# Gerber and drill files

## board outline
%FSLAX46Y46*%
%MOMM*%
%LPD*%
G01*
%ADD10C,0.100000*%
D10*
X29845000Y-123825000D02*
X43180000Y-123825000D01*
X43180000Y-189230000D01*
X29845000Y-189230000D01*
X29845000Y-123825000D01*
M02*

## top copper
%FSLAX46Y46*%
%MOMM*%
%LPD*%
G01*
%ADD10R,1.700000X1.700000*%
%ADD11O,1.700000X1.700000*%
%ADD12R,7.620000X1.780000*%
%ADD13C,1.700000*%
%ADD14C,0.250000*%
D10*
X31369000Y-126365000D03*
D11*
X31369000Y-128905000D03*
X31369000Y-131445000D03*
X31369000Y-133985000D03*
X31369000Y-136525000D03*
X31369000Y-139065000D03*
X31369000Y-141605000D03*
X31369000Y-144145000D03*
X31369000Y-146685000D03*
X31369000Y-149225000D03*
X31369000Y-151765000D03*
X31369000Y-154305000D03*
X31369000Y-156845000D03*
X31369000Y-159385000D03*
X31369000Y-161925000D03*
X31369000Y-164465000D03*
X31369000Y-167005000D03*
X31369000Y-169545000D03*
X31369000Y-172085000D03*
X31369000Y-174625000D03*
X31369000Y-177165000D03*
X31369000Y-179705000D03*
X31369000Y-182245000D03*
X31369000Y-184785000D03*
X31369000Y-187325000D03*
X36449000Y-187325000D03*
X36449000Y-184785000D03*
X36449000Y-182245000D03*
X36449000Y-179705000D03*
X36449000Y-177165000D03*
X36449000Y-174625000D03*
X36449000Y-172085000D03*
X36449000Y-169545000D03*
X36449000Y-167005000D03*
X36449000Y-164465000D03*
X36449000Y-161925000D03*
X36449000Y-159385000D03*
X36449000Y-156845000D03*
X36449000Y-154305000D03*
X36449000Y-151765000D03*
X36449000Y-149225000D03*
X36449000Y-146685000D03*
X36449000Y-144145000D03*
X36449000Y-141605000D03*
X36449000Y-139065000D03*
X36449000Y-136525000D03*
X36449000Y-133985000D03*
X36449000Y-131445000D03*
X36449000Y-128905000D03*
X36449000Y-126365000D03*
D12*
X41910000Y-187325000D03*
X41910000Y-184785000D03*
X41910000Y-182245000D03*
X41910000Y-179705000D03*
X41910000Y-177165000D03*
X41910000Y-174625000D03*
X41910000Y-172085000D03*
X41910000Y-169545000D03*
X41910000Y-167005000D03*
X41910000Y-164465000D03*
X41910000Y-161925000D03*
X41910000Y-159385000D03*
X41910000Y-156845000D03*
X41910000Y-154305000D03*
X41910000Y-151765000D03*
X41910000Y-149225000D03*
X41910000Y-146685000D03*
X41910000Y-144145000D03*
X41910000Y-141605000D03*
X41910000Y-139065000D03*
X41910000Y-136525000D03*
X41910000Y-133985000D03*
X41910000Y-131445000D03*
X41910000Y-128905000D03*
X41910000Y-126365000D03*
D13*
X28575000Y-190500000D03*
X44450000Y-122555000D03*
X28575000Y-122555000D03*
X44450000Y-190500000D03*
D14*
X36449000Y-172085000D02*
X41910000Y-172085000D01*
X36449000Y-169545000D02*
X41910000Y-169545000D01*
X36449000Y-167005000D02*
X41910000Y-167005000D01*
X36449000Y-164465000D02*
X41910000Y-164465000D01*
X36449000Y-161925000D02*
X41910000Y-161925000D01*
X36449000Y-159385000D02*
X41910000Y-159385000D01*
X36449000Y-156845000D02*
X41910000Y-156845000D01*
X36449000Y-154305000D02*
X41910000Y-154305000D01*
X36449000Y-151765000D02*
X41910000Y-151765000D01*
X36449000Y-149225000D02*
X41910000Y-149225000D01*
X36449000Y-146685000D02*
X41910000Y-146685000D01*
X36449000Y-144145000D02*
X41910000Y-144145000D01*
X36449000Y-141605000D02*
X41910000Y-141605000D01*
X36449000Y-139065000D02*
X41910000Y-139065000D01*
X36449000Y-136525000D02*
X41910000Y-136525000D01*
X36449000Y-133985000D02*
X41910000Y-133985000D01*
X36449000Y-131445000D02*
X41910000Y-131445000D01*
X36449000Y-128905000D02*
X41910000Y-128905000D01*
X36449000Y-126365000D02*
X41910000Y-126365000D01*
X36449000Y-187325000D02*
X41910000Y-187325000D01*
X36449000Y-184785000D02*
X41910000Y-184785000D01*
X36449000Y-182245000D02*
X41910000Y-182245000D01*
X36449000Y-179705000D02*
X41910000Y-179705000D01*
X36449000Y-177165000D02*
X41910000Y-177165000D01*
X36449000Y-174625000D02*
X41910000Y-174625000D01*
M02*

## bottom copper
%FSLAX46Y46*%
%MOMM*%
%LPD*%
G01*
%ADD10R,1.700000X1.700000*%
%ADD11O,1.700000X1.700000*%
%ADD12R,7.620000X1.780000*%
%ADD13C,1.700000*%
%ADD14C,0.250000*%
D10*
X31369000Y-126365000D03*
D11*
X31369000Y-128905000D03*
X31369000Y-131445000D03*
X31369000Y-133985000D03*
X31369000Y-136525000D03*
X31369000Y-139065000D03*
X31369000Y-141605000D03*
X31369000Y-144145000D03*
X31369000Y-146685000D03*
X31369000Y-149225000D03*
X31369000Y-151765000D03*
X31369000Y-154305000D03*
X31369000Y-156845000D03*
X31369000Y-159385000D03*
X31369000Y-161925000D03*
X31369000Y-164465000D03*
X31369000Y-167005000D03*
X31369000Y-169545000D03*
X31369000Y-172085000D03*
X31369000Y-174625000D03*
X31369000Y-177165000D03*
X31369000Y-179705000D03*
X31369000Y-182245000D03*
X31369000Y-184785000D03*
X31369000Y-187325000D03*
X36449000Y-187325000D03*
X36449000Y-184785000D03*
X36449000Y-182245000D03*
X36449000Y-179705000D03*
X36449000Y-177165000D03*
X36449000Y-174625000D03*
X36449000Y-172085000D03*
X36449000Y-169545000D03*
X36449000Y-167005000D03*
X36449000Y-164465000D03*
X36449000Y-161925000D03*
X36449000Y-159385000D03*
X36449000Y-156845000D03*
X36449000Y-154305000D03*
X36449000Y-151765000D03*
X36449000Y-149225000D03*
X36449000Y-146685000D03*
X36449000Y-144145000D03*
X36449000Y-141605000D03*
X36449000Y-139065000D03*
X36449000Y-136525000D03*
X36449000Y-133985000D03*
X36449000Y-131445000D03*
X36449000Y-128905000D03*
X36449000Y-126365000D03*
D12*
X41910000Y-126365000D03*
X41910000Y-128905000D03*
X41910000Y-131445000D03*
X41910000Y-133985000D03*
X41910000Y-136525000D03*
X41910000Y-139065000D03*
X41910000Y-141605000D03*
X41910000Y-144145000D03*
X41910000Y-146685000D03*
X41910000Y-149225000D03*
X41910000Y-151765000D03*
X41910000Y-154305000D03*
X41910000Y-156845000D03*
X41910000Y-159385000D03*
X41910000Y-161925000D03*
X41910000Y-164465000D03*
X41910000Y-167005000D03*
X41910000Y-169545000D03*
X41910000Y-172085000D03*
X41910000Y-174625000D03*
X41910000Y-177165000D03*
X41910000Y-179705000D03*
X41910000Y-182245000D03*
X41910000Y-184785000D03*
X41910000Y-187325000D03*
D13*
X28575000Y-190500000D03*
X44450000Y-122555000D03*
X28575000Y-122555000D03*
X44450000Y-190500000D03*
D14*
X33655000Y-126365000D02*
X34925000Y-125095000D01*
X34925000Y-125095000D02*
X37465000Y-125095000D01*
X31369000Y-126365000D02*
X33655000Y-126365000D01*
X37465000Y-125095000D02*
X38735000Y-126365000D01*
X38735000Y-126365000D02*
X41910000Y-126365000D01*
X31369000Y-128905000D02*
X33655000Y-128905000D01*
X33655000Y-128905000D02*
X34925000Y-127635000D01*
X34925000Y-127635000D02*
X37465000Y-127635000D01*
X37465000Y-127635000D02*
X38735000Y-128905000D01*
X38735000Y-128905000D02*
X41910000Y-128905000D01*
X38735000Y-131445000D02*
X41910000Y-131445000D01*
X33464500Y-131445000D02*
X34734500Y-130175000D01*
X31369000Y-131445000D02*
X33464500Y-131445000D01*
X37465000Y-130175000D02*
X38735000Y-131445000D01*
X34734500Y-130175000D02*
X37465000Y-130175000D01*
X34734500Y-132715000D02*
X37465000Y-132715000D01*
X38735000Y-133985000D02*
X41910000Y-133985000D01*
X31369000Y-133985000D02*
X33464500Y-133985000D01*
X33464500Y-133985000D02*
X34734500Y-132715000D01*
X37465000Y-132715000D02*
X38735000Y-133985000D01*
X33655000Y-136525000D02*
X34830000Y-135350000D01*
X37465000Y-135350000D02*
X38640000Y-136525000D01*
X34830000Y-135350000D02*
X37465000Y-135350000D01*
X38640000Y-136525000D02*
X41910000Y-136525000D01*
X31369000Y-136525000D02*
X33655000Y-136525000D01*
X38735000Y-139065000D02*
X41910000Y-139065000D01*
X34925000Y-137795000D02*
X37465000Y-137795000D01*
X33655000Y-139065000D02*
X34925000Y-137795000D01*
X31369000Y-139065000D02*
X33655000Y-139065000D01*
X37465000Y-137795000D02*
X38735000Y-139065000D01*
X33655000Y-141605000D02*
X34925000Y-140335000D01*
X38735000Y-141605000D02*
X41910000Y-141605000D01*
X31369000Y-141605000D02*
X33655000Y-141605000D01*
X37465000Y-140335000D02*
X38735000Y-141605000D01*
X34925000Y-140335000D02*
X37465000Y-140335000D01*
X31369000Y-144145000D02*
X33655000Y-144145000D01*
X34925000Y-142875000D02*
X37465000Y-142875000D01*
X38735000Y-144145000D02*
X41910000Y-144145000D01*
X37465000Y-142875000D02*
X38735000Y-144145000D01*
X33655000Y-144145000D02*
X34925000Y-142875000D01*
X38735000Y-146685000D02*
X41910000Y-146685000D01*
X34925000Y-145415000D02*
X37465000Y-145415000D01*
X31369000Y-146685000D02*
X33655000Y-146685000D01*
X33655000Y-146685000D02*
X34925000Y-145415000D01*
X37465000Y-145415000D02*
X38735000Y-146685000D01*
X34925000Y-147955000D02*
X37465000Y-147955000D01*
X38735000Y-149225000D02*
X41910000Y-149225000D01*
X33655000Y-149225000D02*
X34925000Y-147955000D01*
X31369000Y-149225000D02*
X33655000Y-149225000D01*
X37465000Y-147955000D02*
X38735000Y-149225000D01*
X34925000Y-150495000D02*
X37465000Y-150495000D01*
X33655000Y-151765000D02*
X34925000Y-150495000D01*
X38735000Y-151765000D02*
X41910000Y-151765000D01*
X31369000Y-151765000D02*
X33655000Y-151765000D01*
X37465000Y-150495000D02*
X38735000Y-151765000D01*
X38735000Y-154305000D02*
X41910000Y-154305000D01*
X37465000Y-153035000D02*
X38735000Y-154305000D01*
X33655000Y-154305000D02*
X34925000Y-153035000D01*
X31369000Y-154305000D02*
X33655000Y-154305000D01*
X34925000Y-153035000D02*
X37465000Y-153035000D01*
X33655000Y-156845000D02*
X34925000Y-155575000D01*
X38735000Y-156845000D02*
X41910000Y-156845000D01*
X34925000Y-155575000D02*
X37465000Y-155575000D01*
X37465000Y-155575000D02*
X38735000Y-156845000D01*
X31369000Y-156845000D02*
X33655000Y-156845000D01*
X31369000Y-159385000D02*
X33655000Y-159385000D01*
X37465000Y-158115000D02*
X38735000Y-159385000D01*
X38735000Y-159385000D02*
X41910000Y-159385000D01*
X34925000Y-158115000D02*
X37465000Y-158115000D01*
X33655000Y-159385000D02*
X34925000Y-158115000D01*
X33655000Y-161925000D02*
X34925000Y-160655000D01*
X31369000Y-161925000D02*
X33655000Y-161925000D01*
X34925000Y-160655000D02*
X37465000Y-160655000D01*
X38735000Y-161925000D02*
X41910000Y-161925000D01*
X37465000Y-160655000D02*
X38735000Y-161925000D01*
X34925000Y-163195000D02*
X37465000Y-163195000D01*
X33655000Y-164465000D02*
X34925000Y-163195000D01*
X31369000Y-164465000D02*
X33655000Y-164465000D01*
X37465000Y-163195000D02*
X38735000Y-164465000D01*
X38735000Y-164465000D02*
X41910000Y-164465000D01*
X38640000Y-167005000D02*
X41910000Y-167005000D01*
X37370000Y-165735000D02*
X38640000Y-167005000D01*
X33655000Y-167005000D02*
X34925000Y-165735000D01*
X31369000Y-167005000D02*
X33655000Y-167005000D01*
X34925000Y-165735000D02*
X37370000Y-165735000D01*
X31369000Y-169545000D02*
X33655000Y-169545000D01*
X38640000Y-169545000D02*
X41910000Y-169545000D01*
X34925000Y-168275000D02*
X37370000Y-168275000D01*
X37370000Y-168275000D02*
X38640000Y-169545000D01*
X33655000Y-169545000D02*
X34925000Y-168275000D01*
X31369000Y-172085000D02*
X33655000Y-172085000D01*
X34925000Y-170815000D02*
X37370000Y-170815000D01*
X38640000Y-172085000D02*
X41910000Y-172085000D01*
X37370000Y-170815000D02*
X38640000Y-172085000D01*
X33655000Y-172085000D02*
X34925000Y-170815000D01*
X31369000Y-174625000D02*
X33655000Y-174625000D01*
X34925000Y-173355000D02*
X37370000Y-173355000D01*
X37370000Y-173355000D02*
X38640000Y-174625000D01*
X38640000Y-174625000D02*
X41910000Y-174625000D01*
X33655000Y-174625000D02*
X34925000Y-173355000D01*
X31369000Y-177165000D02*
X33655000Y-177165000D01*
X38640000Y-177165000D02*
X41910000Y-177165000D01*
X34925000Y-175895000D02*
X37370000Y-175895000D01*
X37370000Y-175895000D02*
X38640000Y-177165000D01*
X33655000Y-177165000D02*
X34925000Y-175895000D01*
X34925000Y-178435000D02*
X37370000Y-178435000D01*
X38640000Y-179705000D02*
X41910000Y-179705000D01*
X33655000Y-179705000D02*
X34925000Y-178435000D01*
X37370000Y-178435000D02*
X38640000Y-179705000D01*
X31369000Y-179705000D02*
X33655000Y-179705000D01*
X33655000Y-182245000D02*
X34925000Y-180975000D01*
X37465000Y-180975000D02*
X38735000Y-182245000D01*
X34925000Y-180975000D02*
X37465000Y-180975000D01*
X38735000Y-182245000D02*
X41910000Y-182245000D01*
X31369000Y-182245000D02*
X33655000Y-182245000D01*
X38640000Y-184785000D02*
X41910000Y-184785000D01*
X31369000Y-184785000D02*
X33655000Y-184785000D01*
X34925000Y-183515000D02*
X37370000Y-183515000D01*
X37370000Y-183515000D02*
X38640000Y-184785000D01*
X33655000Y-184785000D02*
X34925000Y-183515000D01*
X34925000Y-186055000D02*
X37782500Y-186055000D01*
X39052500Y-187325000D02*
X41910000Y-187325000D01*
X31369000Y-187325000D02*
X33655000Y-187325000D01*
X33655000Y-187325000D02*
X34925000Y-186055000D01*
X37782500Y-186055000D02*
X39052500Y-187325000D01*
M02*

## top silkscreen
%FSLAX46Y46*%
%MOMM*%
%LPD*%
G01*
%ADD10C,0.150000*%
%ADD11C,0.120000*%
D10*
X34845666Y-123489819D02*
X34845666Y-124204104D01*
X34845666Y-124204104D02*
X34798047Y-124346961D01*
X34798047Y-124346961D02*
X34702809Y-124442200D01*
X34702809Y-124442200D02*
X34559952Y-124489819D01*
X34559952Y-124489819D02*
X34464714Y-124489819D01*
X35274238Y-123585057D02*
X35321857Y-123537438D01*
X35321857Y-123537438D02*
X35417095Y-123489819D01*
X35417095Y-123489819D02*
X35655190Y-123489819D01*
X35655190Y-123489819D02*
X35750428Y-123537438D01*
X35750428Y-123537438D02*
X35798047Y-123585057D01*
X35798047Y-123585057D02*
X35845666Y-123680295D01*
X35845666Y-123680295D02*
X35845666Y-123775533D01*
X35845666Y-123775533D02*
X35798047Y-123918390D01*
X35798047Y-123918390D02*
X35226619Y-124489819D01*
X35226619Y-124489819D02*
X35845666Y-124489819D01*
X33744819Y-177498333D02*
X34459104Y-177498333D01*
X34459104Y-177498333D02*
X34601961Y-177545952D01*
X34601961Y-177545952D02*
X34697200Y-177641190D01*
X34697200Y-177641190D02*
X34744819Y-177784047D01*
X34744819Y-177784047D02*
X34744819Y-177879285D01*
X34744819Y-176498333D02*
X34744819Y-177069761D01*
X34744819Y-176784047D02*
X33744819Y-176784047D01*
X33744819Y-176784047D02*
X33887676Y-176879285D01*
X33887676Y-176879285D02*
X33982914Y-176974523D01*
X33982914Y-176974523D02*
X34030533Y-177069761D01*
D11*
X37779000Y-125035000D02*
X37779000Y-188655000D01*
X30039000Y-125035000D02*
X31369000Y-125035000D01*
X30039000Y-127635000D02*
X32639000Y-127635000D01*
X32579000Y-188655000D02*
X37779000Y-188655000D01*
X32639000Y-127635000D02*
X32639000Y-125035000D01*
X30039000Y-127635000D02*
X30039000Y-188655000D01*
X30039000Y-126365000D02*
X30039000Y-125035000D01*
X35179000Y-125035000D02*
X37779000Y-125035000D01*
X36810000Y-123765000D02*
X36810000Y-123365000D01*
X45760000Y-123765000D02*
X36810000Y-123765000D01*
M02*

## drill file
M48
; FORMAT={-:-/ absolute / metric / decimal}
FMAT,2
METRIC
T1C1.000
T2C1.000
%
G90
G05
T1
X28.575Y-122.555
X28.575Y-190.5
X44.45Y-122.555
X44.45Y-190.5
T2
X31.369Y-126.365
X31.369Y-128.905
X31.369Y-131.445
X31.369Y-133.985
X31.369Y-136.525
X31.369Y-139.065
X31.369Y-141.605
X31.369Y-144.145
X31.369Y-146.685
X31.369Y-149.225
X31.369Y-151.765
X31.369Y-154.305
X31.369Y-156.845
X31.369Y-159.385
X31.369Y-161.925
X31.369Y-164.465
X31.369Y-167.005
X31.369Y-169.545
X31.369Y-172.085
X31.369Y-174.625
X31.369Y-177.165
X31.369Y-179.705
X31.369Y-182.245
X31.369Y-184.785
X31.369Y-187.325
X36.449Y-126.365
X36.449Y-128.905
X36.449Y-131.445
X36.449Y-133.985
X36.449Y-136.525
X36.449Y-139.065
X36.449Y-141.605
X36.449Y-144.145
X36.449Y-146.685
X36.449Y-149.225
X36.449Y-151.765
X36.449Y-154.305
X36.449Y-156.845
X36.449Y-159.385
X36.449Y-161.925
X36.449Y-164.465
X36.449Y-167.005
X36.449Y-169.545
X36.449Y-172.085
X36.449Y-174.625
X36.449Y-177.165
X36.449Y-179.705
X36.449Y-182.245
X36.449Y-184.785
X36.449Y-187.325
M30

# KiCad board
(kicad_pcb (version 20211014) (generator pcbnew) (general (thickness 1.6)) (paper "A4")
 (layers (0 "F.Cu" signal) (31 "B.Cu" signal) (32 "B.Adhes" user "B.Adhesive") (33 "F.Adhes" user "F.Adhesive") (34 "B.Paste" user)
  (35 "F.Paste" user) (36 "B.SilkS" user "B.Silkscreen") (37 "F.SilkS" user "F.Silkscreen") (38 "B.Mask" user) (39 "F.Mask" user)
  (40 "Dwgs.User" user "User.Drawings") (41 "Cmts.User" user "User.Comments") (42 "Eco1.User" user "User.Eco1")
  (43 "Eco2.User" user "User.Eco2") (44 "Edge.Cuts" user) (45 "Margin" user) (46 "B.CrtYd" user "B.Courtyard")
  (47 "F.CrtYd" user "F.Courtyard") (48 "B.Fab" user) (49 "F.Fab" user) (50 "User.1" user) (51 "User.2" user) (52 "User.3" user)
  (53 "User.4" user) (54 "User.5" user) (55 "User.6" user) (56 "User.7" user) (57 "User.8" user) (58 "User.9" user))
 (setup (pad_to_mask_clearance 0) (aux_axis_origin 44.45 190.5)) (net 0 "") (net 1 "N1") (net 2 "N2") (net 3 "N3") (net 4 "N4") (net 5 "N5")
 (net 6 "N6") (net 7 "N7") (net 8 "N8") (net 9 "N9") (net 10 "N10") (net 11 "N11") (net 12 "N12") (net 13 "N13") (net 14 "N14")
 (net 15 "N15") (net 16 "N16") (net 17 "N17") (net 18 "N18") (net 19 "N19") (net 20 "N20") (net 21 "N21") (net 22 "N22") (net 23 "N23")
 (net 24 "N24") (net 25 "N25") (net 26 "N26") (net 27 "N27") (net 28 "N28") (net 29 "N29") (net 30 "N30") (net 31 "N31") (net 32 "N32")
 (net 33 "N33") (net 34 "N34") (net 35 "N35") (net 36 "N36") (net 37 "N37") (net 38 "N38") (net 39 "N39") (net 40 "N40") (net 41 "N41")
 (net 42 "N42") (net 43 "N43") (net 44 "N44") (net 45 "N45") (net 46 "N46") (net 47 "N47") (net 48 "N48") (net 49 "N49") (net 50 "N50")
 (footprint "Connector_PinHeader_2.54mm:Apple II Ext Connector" (layer "F.Cu") (at 31.369 126.365)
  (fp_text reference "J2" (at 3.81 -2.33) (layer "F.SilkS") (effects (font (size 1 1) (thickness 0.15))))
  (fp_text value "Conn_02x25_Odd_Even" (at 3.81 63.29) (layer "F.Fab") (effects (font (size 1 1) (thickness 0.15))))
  (fp_line (start 6.41 -1.33) (end 6.41 62.29) (layer "F.SilkS") (width 0.12))
  (fp_line (start -1.33 -1.33) (end 0 -1.33) (layer "F.SilkS") (width 0.12))
  (fp_line (start -1.33 1.27) (end 1.27 1.27) (layer "F.SilkS") (width 0.12))
  (fp_line (start 1.21 62.29) (end 6.41 62.29) (layer "F.SilkS") (width 0.12))
  (fp_line (start 1.27 1.27) (end 1.27 -1.33) (layer "F.SilkS") (width 0.12))
  (fp_line (start -1.33 1.27) (end -1.33 62.29) (layer "F.SilkS") (width 0.12))
  (fp_line (start -1.33 0) (end -1.33 -1.33) (layer "F.SilkS") (width 0.12))
  (fp_line (start 3.81 -1.33) (end 6.41 -1.33) (layer "F.SilkS") (width 0.12))
  (pad "1" thru_hole rect (at 0 0) (size 1.7 1.7) (drill 1) (layers *.Cu *.Mask) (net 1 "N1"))
  (pad "2" thru_hole oval (at 0 2.54) (size 1.7 1.7) (drill 1) (layers *.Cu *.Mask) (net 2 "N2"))
  (pad "3" thru_hole oval (at 0 5.08) (size 1.7 1.7) (drill 1) (layers *.Cu *.Mask) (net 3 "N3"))
  (pad "4" thru_hole oval (at 0 7.62) (size 1.7 1.7) (drill 1) (layers *.Cu *.Mask) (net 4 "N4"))
  (pad "5" thru_hole oval (at 0 10.16) (size 1.7 1.7) (drill 1) (layers *.Cu *.Mask) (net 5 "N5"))
  (pad "6" thru_hole oval (at 0 12.7) (size 1.7 1.7) (drill 1) (layers *.Cu *.Mask) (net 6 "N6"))
  (pad "7" thru_hole oval (at 0 15.24) (size 1.7 1.7) (drill 1) (layers *.Cu *.Mask) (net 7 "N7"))
  (pad "8" thru_hole oval (at 0 17.78) (size 1.7 1.7) (drill 1) (layers *.Cu *.Mask) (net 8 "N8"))
  (pad "9" thru_hole oval (at 0 20.32) (size 1.7 1.7) (drill 1) (layers *.Cu *.Mask) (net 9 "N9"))
  (pad "10" thru_hole oval (at 0 22.86) (size 1.7 1.7) (drill 1) (layers *.Cu *.Mask) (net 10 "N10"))
  (pad "11" thru_hole oval (at 0 25.4) (size 1.7 1.7) (drill 1) (layers *.Cu *.Mask) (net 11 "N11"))
  (pad "12" thru_hole oval (at 0 27.94) (size 1.7 1.7) (drill 1) (layers *.Cu *.Mask) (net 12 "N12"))
  (pad "13" thru_hole oval (at 0 30.48) (size 1.7 1.7) (drill 1) (layers *.Cu *.Mask) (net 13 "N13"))
  (pad "14" thru_hole oval (at 0 33.02) (size 1.7 1.7) (drill 1) (layers *.Cu *.Mask) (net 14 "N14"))
  (pad "15" thru_hole oval (at 0 35.56) (size 1.7 1.7) (drill 1) (layers *.Cu *.Mask) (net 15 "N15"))
  (pad "16" thru_hole oval (at 0 38.1) (size 1.7 1.7) (drill 1) (layers *.Cu *.Mask) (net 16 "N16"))
  (pad "17" thru_hole oval (at 0 40.64) (size 1.7 1.7) (drill 1) (layers *.Cu *.Mask) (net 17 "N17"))
  (pad "18" thru_hole oval (at 0 43.18) (size 1.7 1.7) (drill 1) (layers *.Cu *.Mask) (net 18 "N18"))
  (pad "19" thru_hole oval (at 0 45.72) (size 1.7 1.7) (drill 1) (layers *.Cu *.Mask) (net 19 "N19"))
  (pad "20" thru_hole oval (at 0 48.26) (size 1.7 1.7) (drill 1) (layers *.Cu *.Mask) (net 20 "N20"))
  (pad "21" thru_hole oval (at 0 50.8) (size 1.7 1.7) (drill 1) (layers *.Cu *.Mask) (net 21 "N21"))
  (pad "22" thru_hole oval (at 0 53.34) (size 1.7 1.7) (drill 1) (layers *.Cu *.Mask) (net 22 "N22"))
  (pad "23" thru_hole oval (at 0 55.88) (size 1.7 1.7) (drill 1) (layers *.Cu *.Mask) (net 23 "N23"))
  (pad "24" thru_hole oval (at 0 58.42) (size 1.7 1.7) (drill 1) (layers *.Cu *.Mask) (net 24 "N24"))
  (pad "25" thru_hole oval (at 0 60.96) (size 1.7 1.7) (drill 1) (layers *.Cu *.Mask) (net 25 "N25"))
  (pad "26" thru_hole oval (at 5.08 60.96 180) (size 1.7 1.7) (drill 1) (layers *.Cu *.Mask) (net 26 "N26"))
  (pad "27" thru_hole oval (at 5.08 58.42 180) (size 1.7 1.7) (drill 1) (layers *.Cu *.Mask) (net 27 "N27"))
  (pad "28" thru_hole oval (at 5.08 55.88 180) (size 1.7 1.7) (drill 1) (layers *.Cu *.Mask) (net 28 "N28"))
  (pad "29" thru_hole oval (at 5.08 53.34 180) (size 1.7 1.7) (drill 1) (layers *.Cu *.Mask) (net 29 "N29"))
  (pad "30" thru_hole oval (at 5.08 50.8 180) (size 1.7 1.7) (drill 1) (layers *.Cu *.Mask) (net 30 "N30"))
  (pad "31" thru_hole oval (at 5.08 48.26 180) (size 1.7 1.7) (drill 1) (layers *.Cu *.Mask) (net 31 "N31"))
  (pad "32" thru_hole oval (at 5.08 45.72 180) (size 1.7 1.7) (drill 1) (layers *.Cu *.Mask) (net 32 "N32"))
  (pad "33" thru_hole oval (at 5.08 43.18 180) (size 1.7 1.7) (drill 1) (layers *.Cu *.Mask) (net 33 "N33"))
  (pad "34" thru_hole oval (at 5.08 40.64 180) (size 1.7 1.7) (drill 1) (layers *.Cu *.Mask) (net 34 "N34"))
  (pad "35" thru_hole oval (at 5.08 38.1 180) (size 1.7 1.7) (drill 1) (layers *.Cu *.Mask) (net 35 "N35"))
  (pad "36" thru_hole oval (at 5.08 35.56 180) (size 1.7 1.7) (drill 1) (layers *.Cu *.Mask) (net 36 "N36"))
  (pad "37" thru_hole oval (at 5.08 33.02 180) (size 1.7 1.7) (drill 1) (layers *.Cu *.Mask) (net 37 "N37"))
  (pad "38" thru_hole oval (at 5.08 30.48 180) (size 1.7 1.7) (drill 1) (layers *.Cu *.Mask) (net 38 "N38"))
  (pad "39" thru_hole oval (at 5.08 27.94 180) (size 1.7 1.7) (drill 1) (layers *.Cu *.Mask) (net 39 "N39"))
  (pad "40" thru_hole oval (at 5.08 25.4 180) (size 1.7 1.7) (drill 1) (layers *.Cu *.Mask) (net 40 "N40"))
  (pad "41" thru_hole oval (at 5.08 22.86 180) (size 1.7 1.7) (drill 1) (layers *.Cu *.Mask) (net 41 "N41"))
  (pad "42" thru_hole oval (at 5.08 20.32 180) (size 1.7 1.7) (drill 1) (layers *.Cu *.Mask) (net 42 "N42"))
  (pad "43" thru_hole oval (at 5.08 17.78 180) (size 1.7 1.7) (drill 1) (layers *.Cu *.Mask) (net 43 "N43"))
  (pad "44" thru_hole oval (at 5.08 15.24 180) (size 1.7 1.7) (drill 1) (layers *.Cu *.Mask) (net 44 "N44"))
  (pad "45" thru_hole oval (at 5.08 12.7 180) (size 1.7 1.7) (drill 1) (layers *.Cu *.Mask) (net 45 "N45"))
  (pad "46" thru_hole oval (at 5.08 10.16 180) (size 1.7 1.7) (drill 1) (layers *.Cu *.Mask) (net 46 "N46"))
  (pad "47" thru_hole oval (at 5.08 7.62 180) (size 1.7 1.7) (drill 1) (layers *.Cu *.Mask) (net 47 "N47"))
  (pad "48" thru_hole oval (at 5.08 5.08 180) (size 1.7 1.7) (drill 1) (layers *.Cu *.Mask) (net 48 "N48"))
  (pad "49" thru_hole oval (at 5.08 2.54 180) (size 1.7 1.7) (drill 1) (layers *.Cu *.Mask) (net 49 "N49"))
  (pad "50" thru_hole oval (at 5.08 0 180) (size 1.7 1.7) (drill 1) (layers *.Cu *.Mask) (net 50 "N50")))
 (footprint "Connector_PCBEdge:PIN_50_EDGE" (layer "F.Cu") (at 41.91 126.365 90)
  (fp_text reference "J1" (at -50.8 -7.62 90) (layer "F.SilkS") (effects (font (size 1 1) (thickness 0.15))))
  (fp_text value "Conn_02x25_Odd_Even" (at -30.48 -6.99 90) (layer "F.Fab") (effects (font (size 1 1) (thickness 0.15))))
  (fp_line (start 2.6 -5.1) (end 3 -5.1) (layer "F.SilkS") (width 0.12))
  (fp_line (start 2.6 3.85) (end 2.6 -5.1) (layer "F.SilkS") (width 0.12))
  (pad "1" connect rect (at 0 0 90) (size 1.78 7.62) (layers "B.Cu" "B.Mask") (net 1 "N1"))
  (pad "2" connect rect (at -2.54 0 90) (size 1.78 7.62) (layers "B.Cu" "B.Mask") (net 2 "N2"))
  (pad "3" connect rect (at -5.08 0 90) (size 1.78 7.62) (layers "B.Cu" "B.Mask") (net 3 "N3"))
  (pad "4" connect rect (at -7.62 0 90) (size 1.78 7.62) (layers "B.Cu" "B.Mask") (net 4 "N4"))
  (pad "5" connect rect (at -10.16 0 90) (size 1.78 7.62) (layers "B.Cu" "B.Mask") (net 5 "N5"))
  (pad "6" connect rect (at -12.7 0 90) (size 1.78 7.62) (layers "B.Cu" "B.Mask") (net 6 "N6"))
  (pad "7" connect rect (at -15.24 0 90) (size 1.78 7.62) (layers "B.Cu" "B.Mask") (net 7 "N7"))
  (pad "8" connect rect (at -17.78 0 90) (size 1.78 7.62) (layers "B.Cu" "B.Mask") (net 8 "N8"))
  (pad "9" connect rect (at -20.32 0 90) (size 1.78 7.62) (layers "B.Cu" "B.Mask") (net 9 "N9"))
  (pad "10" connect rect (at -22.86 0 90) (size 1.78 7.62) (layers "B.Cu" "B.Mask") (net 10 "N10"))
  (pad "11" connect rect (at -25.4 0 90) (size 1.78 7.62) (layers "B.Cu" "B.Mask") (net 11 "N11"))
  (pad "12" connect rect (at -27.94 0 90) (size 1.78 7.62) (layers "B.Cu" "B.Mask") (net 12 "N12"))
  (pad "13" connect rect (at -30.48 0 90) (size 1.78 7.62) (layers "B.Cu" "B.Mask") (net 13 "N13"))
  (pad "14" connect rect (at -33.02 0 90) (size 1.78 7.62) (layers "B.Cu" "B.Mask") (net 14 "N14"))
  (pad "15" connect rect (at -35.56 0 90) (size 1.78 7.62) (layers "B.Cu" "B.Mask") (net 15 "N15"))
  (pad "16" connect rect (at -38.1 0 90) (size 1.78 7.62) (layers "B.Cu" "B.Mask") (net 16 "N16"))
  (pad "17" connect rect (at -40.64 0 90) (size 1.78 7.62) (layers "B.Cu" "B.Mask") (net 17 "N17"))
  (pad "18" connect rect (at -43.18 0 90) (size 1.78 7.62) (layers "B.Cu" "B.Mask") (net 18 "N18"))
  (pad "19" connect rect (at -45.72 0 90) (size 1.78 7.62) (layers "B.Cu" "B.Mask") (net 19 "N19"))
  (pad "20" connect rect (at -48.26 0 90) (size 1.78 7.62) (layers "B.Cu" "B.Mask") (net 20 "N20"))
  (pad "21" connect rect (at -50.8 0 90) (size 1.78 7.62) (layers "B.Cu" "B.Mask") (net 21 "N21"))
  (pad "22" connect rect (at -53.34 0 90) (size 1.78 7.62) (layers "B.Cu" "B.Mask") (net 22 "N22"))
  (pad "23" connect rect (at -55.88 0 90) (size 1.78 7.62) (layers "B.Cu" "B.Mask") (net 23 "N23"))
  (pad "24" connect rect (at -58.42 0 90) (size 1.78 7.62) (layers "B.Cu" "B.Mask") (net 24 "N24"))
  (pad "25" connect rect (at -60.96 0 90) (size 1.78 7.62) (layers "B.Cu" "B.Mask") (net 25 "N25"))
  (pad "26" connect rect (at -60.96 0 90) (size 1.78 7.62) (layers "F.Cu" "F.Mask") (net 26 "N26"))
  (pad "27" connect rect (at -58.42 0 90) (size 1.78 7.62) (layers "F.Cu" "F.Mask") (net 27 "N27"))
  (pad "28" connect rect (at -55.88 0 90) (size 1.78 7.62) (layers "F.Cu" "F.Mask") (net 28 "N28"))
  (pad "29" connect rect (at -53.34 0 90) (size 1.78 7.62) (layers "F.Cu" "F.Mask") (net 29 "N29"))
  (pad "30" connect rect (at -50.8 0 90) (size 1.78 7.62) (layers "F.Cu" "F.Mask") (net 30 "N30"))
  (pad "31" connect rect (at -48.26 0 90) (size 1.78 7.62) (layers "F.Cu" "F.Mask") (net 31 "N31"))
  (pad "32" connect rect (at -45.72 0 90) (size 1.78 7.62) (layers "F.Cu" "F.Mask") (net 32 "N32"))
  (pad "33" connect rect (at -43.18 0 90) (size 1.78 7.62) (layers "F.Cu" "F.Mask") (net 33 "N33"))
  (pad "34" connect rect (at -40.64 0 90) (size 1.78 7.62) (layers "F.Cu" "F.Mask") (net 34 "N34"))
  (pad "35" connect rect (at -38.1 0 90) (size 1.78 7.62) (layers "F.Cu" "F.Mask") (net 35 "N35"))
  (pad "36" connect rect (at -35.56 0 90) (size 1.78 7.62) (layers "F.Cu" "F.Mask") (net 36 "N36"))
  (pad "37" connect rect (at -33.02 0 90) (size 1.78 7.62) (layers "F.Cu" "F.Mask") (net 37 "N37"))
  (pad "38" connect rect (at -30.48 0 90) (size 1.78 7.62) (layers "F.Cu" "F.Mask") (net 38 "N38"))
  (pad "39" connect rect (at -27.94 0 90) (size 1.78 7.62) (layers "F.Cu" "F.Mask") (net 39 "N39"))
  (pad "40" connect rect (at -25.4 0 90) (size 1.78 7.62) (layers "F.Cu" "F.Mask") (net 40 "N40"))
  (pad "41" connect rect (at -22.86 0 90) (size 1.78 7.62) (layers "F.Cu" "F.Mask") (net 41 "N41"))
  (pad "42" connect rect (at -20.32 0 90) (size 1.78 7.62) (layers "F.Cu" "F.Mask") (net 42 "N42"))
  (pad "43" connect rect (at -17.78 0 90) (size 1.78 7.62) (layers "F.Cu" "F.Mask") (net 43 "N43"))
  (pad "44" connect rect (at -15.24 0 90) (size 1.78 7.62) (layers "F.Cu" "F.Mask") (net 44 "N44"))
  (pad "45" connect rect (at -12.7 0 90) (size 1.78 7.62) (layers "F.Cu" "F.Mask") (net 45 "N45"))
  (pad "46" connect rect (at -10.16 0 90) (size 1.78 7.62) (layers "F.Cu" "F.Mask") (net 46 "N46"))
  (pad "47" connect rect (at -7.62 0 90) (size 1.78 7.62) (layers "F.Cu" "F.Mask") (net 47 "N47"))
  (pad "48" connect rect (at -5.08 0 90) (size 1.78 7.62) (layers "F.Cu" "F.Mask") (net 48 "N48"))
  (pad "49" connect rect (at -2.54 0 90) (size 1.78 7.62) (layers "F.Cu" "F.Mask") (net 49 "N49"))
  (pad "50" connect rect (at 0 0 90) (size 1.78 7.62) (layers "F.Cu" "F.Mask") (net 50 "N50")))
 (gr_rect (start 29.845 123.825) (end 43.18 189.23) (layer "Edge.Cuts") (width 0.1) (fill none))
 (via (at 28.575 190.5) (size 1.7) (drill 1) (layers "F.Cu" "B.Cu") (free) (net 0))
 (via (at 44.45 122.555) (size 1.7) (drill 1) (layers "F.Cu" "B.Cu") (free) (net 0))
 (via (at 28.575 122.555) (size 1.7) (drill 1) (layers "F.Cu" "B.Cu") (free) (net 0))
 (via (at 44.45 190.5) (size 1.7) (drill 1) (layers "F.Cu" "B.Cu") (free) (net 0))
 (segment (start 33.655 126.365) (end 34.925 125.095) (width 0.25) (layer "B.Cu") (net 1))
 (segment (start 34.925 125.095) (end 37.465 125.095) (width 0.25) (layer "B.Cu") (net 1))
 (segment (start 31.369 126.365) (end 33.655 126.365) (width 0.25) (layer "B.Cu") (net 1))
 (segment (start 37.465 125.095) (end 38.735 126.365) (width 0.25) (layer "B.Cu") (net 1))
 (segment (start 38.735 126.365) (end 41.91 126.365) (width 0.25) (layer "B.Cu") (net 1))
 (segment (start 31.369 128.905) (end 33.655 128.905) (width 0.25) (layer "B.Cu") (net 2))
 (segment (start 33.655 128.905) (end 34.925 127.635) (width 0.25) (layer "B.Cu") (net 2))
 (segment (start 34.925 127.635) (end 37.465 127.635) (width 0.25) (layer "B.Cu") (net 2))
 (segment (start 37.465 127.635) (end 38.735 128.905) (width 0.25) (layer "B.Cu") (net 2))
 (segment (start 38.735 128.905) (end 41.91 128.905) (width 0.25) (layer "B.Cu") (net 2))
 (segment (start 38.735 131.445) (end 41.91 131.445) (width 0.25) (layer "B.Cu") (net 3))
 (segment (start 33.4645 131.445) (end 34.7345 130.175) (width 0.25) (layer "B.Cu") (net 3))
 (segment (start 31.369 131.445) (end 33.4645 131.445) (width 0.25) (layer "B.Cu") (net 3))
 (segment (start 37.465 130.175) (end 38.735 131.445) (width 0.25) (layer "B.Cu") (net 3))
 (segment (start 34.7345 130.175) (end 37.465 130.175) (width 0.25) (layer "B.Cu") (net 3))
 (segment (start 34.7345 132.715) (end 37.465 132.715) (width 0.25) (layer "B.Cu") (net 4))
 (segment (start 38.735 133.985) (end 41.91 133.985) (width 0.25) (layer "B.Cu") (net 4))
 (segment (start 31.369 133.985) (end 33.4645 133.985) (width 0.25) (layer "B.Cu") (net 4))
 (segment (start 33.4645 133.985) (end 34.7345 132.715) (width 0.25) (layer "B.Cu") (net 4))
 (segment (start 37.465 132.715) (end 38.735 133.985) (width 0.25) (layer "B.Cu") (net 4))
 (segment (start 33.655 136.525) (end 34.83 135.35) (width 0.25) (layer "B.Cu") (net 5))
 (segment (start 37.465 135.35) (end 38.64 136.525) (width 0.25) (layer "B.Cu") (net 5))
 (segment (start 34.83 135.35) (end 37.465 135.35) (width 0.25) (layer "B.Cu") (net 5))
 (segment (start 38.64 136.525) (end 41.91 136.525) (width 0.25) (layer "B.Cu") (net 5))
 (segment (start 31.369 136.525) (end 33.655 136.525) (width 0.25) (layer "B.Cu") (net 5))
 (segment (start 38.735 139.065) (end 41.91 139.065) (width 0.25) (layer "B.Cu") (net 6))
 (segment (start 34.925 137.795) (end 37.465 137.795) (width 0.25) (layer "B.Cu") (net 6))
 (segment (start 33.655 139.065) (end 34.925 137.795) (width 0.25) (layer "B.Cu") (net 6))
 (segment (start 31.369 139.065) (end 33.655 139.065) (width 0.25) (layer "B.Cu") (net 6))
 (segment (start 37.465 137.795) (end 38.735 139.065) (width 0.25) (layer "B.Cu") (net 6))
 (segment (start 33.655 141.605) (end 34.925 140.335) (width 0.25) (layer "B.Cu") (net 7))
 (segment (start 38.735 141.605) (end 41.91 141.605) (width 0.25) (layer "B.Cu") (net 7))
 (segment (start 31.369 141.605) (end 33.655 141.605) (width 0.25) (layer "B.Cu") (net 7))
 (segment (start 37.465 140.335) (end 38.735 141.605) (width 0.25) (layer "B.Cu") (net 7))
 (segment (start 34.925 140.335) (end 37.465 140.335) (width 0.25) (layer "B.Cu") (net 7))
 (segment (start 31.369 144.145) (end 33.655 144.145) (width 0.25) (layer "B.Cu") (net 8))
 (segment (start 34.925 142.875) (end 37.465 142.875) (width 0.25) (layer "B.Cu") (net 8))
 (segment (start 38.735 144.145) (end 41.91 144.145) (width 0.25) (layer "B.Cu") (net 8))
 (segment (start 37.465 142.875) (end 38.735 144.145) (width 0.25) (layer "B.Cu") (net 8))
 (segment (start 33.655 144.145) (end 34.925 142.875) (width 0.25) (layer "B.Cu") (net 8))
 (segment (start 38.735 146.685) (end 41.91 146.685) (width 0.25) (layer "B.Cu") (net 9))
 (segment (start 34.925 145.415) (end 37.465 145.415) (width 0.25) (layer "B.Cu") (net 9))
 (segment (start 31.369 146.685) (end 33.655 146.685) (width 0.25) (layer "B.Cu") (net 9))
 (segment (start 33.655 146.685) (end 34.925 145.415) (width 0.25) (layer "B.Cu") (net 9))
 (segment (start 37.465 145.415) (end 38.735 146.685) (width 0.25) (layer "B.Cu") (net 9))
 (segment (start 34.925 147.955) (end 37.465 147.955) (width 0.25) (layer "B.Cu") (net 10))
 (segment (start 38.735 149.225) (end 41.91 149.225) (width 0.25) (layer "B.Cu") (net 10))
 (segment (start 33.655 149.225) (end 34.925 147.955) (width 0.25) (layer "B.Cu") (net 10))
 (segment (start 31.369 149.225) (end 33.655 149.225) (width 0.25) (layer "B.Cu") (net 10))
 (segment (start 37.465 147.955) (end 38.735 149.225) (width 0.25) (layer "B.Cu") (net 10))
 (segment (start 34.925 150.495) (end 37.465 150.495) (width 0.25) (layer "B.Cu") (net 11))
 (segment (start 33.655 151.765) (end 34.925 150.495) (width 0.25) (layer "B.Cu") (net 11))
 (segment (start 38.735 151.765) (end 41.91 151.765) (width 0.25) (layer "B.Cu") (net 11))
 (segment (start 31.369 151.765) (end 33.655 151.765) (width 0.25) (layer "B.Cu") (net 11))
 (segment (start 37.465 150.495) (end 38.735 151.765) (width 0.25) (layer "B.Cu") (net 11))
 (segment (start 38.735 154.305) (end 41.91 154.305) (width 0.25) (layer "B.Cu") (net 12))
 (segment (start 37.465 153.035) (end 38.735 154.305) (width 0.25) (layer "B.Cu") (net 12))
 (segment (start 33.655 154.305) (end 34.925 153.035) (width 0.25) (layer "B.Cu") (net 12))
 (segment (start 31.369 154.305) (end 33.655 154.305) (width 0.25) (layer "B.Cu") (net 12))
 (segment (start 34.925 153.035) (end 37.465 153.035) (width 0.25) (layer "B.Cu") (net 12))
 (segment (start 33.655 156.845) (end 34.925 155.575) (width 0.25) (layer "B.Cu") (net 13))
 (segment (start 38.735 156.845) (end 41.91 156.845) (width 0.25) (layer "B.Cu") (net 13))
 (segment (start 34.925 155.575) (end 37.465 155.575) (width 0.25) (layer "B.Cu") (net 13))
 (segment (start 37.465 155.575) (end 38.735 156.845) (width 0.25) (layer "B.Cu") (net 13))
 (segment (start 31.369 156.845) (end 33.655 156.845) (width 0.25) (layer "B.Cu") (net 13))
 (segment (start 31.369 159.385) (end 33.655 159.385) (width 0.25) (layer "B.Cu") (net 14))
 (segment (start 37.465 158.115) (end 38.735 159.385) (width 0.25) (layer "B.Cu") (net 14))
 (segment (start 38.735 159.385) (end 41.91 159.385) (width 0.25) (layer "B.Cu") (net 14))
 (segment (start 34.925 158.115) (end 37.465 158.115) (width 0.25) (layer "B.Cu") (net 14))
 (segment (start 33.655 159.385) (end 34.925 158.115) (width 0.25) (layer "B.Cu") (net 14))
 (segment (start 33.655 161.925) (end 34.925 160.655) (width 0.25) (layer "B.Cu") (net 15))
 (segment (start 31.369 161.925) (end 33.655 161.925) (width 0.25) (layer "B.Cu") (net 15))
 (segment (start 34.925 160.655) (end 37.465 160.655) (width 0.25) (layer "B.Cu") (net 15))
 (segment (start 38.735 161.925) (end 41.91 161.925) (width 0.25) (layer "B.Cu") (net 15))
 (segment (start 37.465 160.655) (end 38.735 161.925) (width 0.25) (layer "B.Cu") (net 15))
 (segment (start 34.925 163.195) (end 37.465 163.195) (width 0.25) (layer "B.Cu") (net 16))
 (segment (start 33.655 164.465) (end 34.925 163.195) (width 0.25) (layer "B.Cu") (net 16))
 (segment (start 31.369 164.465) (end 33.655 164.465) (width 0.25) (layer "B.Cu") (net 16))
 (segment (start 37.465 163.195) (end 38.735 164.465) (width 0.25) (layer "B.Cu") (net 16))
 (segment (start 38.735 164.465) (end 41.91 164.465) (width 0.25) (layer "B.Cu") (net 16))
 (segment (start 38.64 167.005) (end 41.91 167.005) (width 0.25) (layer "B.Cu") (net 17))
 (segment (start 37.37 165.735) (end 38.64 167.005) (width 0.25) (layer "B.Cu") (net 17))
 (segment (start 33.655 167.005) (end 34.925 165.735) (width 0.25) (layer "B.Cu") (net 17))
 (segment (start 31.369 167.005) (end 33.655 167.005) (width 0.25) (layer "B.Cu") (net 17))
 (segment (start 34.925 165.735) (end 37.37 165.735) (width 0.25) (layer "B.Cu") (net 17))
 (segment (start 31.369 169.545) (end 33.655 169.545) (width 0.25) (layer "B.Cu") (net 18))
 (segment (start 38.64 169.545) (end 41.91 169.545) (width 0.25) (layer "B.Cu") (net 18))
 (segment (start 34.925 168.275) (end 37.37 168.275) (width 0.25) (layer "B.Cu") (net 18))
 (segment (start 37.37 168.275) (end 38.64 169.545) (width 0.25) (layer "B.Cu") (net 18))
 (segment (start 33.655 169.545) (end 34.925 168.275) (width 0.25) (layer "B.Cu") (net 18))
 (segment (start 31.369 172.085) (end 33.655 172.085) (width 0.25) (layer "B.Cu") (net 19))
 (segment (start 34.925 170.815) (end 37.37 170.815) (width 0.25) (layer "B.Cu") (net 19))
 (segment (start 38.64 172.085) (end 41.91 172.085) (width 0.25) (layer "B.Cu") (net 19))
 (segment (start 37.37 170.815) (end 38.64 172.085) (width 0.25) (layer "B.Cu") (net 19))
 (segment (start 33.655 172.085) (end 34.925 170.815) (width 0.25) (layer "B.Cu") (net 19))
 (segment (start 31.369 174.625) (end 33.655 174.625) (width 0.25) (layer "B.Cu") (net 20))
 (segment (start 34.925 173.355) (end 37.37 173.355) (width 0.25) (layer "B.Cu") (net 20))
 (segment (start 37.37 173.355) (end 38.64 174.625) (width 0.25) (layer "B.Cu") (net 20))
 (segment (start 38.64 174.625) (end 41.91 174.625) (width 0.25) (layer "B.Cu") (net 20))
 (segment (start 33.655 174.625) (end 34.925 173.355) (width 0.25) (layer "B.Cu") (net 20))
 (segment (start 31.369 177.165) (end 33.655 177.165) (width 0.25) (layer "B.Cu") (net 21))
 (segment (start 38.64 177.165) (end 41.91 177.165) (width 0.25) (layer "B.Cu") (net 21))
 (segment (start 34.925 175.895) (end 37.37 175.895) (width 0.25) (layer "B.Cu") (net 21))
 (segment (start 37.37 175.895) (end 38.64 177.165) (width 0.25) (layer "B.Cu") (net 21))
 (segment (start 33.655 177.165) (end 34.925 175.895) (width 0.25) (layer "B.Cu") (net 21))
 (segment (start 34.925 178.435) (end 37.37 178.435) (width 0.25) (layer "B.Cu") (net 22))
 (segment (start 38.64 179.705) (end 41.91 179.705) (width 0.25) (layer "B.Cu") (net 22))
 (segment (start 33.655 179.705) (end 34.925 178.435) (width 0.25) (layer "B.Cu") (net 22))
 (segment (start 37.37 178.435) (end 38.64 179.705) (width 0.25) (layer "B.Cu") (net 22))
 (segment (start 31.369 179.705) (end 33.655 179.705) (width 0.25) (layer "B.Cu") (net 22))
 (segment (start 33.655 182.245) (end 34.925 180.975) (width 0.25) (layer "B.Cu") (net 23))
 (segment (start 37.465 180.975) (end 38.735 182.245) (width 0.25) (layer "B.Cu") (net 23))
 (segment (start 34.925 180.975) (end 37.465 180.975) (width 0.25) (layer "B.Cu") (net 23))
 (segment (start 38.735 182.245) (end 41.91 182.245) (width 0.25) (layer "B.Cu") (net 23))
 (segment (start 31.369 182.245) (end 33.655 182.245) (width 0.25) (layer "B.Cu") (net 23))
 (segment (start 38.64 184.785) (end 41.91 184.785) (width 0.25) (layer "B.Cu") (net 24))
 (segment (start 31.369 184.785) (end 33.655 184.785) (width 0.25) (layer "B.Cu") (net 24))
 (segment (start 34.925 183.515) (end 37.37 183.515) (width 0.25) (layer "B.Cu") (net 24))
 (segment (start 37.37 183.515) (end 38.64 184.785) (width 0.25) (layer "B.Cu") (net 24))
 (segment (start 33.655 184.785) (end 34.925 183.515) (width 0.25) (layer "B.Cu") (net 24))
 (segment (start 34.925 186.055) (end 37.7825 186.055) (width 0.25) (layer "B.Cu") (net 25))
 (segment (start 39.0525 187.325) (end 41.91 187.325) (width 0.25) (layer "B.Cu") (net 25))
 (segment (start 31.369 187.325) (end 33.655 187.325) (width 0.25) (layer "B.Cu") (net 25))
 (segment (start 33.655 187.325) (end 34.925 186.055) (width 0.25) (layer "B.Cu") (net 25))
 (segment (start 37.7825 186.055) (end 39.0525 187.325) (width 0.25) (layer "B.Cu") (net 25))
 (segment (start 36.449 172.085) (end 41.91 172.085) (width 0.25) (layer "F.Cu") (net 32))
 (segment (start 36.449 169.545) (end 41.91 169.545) (width 0.25) (layer "F.Cu") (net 33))
 (segment (start 36.449 167.005) (end 41.91 167.005) (width 0.25) (layer "F.Cu") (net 34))
 (segment (start 36.449 164.465) (end 41.91 164.465) (width 0.25) (layer "F.Cu") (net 35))
 (segment (start 36.449 161.925) (end 41.91 161.925) (width 0.25) (layer "F.Cu") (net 36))
 (segment (start 36.449 159.385) (end 41.91 159.385) (width 0.25) (layer "F.Cu") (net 37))
 (segment (start 36.449 156.845) (end 41.91 156.845) (width 0.25) (layer "F.Cu") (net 38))
 (segment (start 36.449 154.305) (end 41.91 154.305) (width 0.25) (layer "F.Cu") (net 39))
 (segment (start 36.449 151.765) (end 41.91 151.765) (width 0.25) (layer "F.Cu") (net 40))
 (segment (start 36.449 149.225) (end 41.91 149.225) (width 0.25) (layer "F.Cu") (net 41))
 (segment (start 36.449 146.685) (end 41.91 146.685) (width 0.25) (layer "F.Cu") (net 42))
 (segment (start 36.449 144.145) (end 41.91 144.145) (width 0.25) (layer "F.Cu") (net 43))
 (segment (start 36.449 141.605) (end 41.91 141.605) (width 0.25) (layer "F.Cu") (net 44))
 (segment (start 36.449 139.065) (end 41.91 139.065) (width 0.25) (layer "F.Cu") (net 45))
 (segment (start 36.449 136.525) (end 41.91 136.525) (width 0.25) (layer "F.Cu") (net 46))
 (segment (start 36.449 133.985) (end 41.91 133.985) (width 0.25) (layer "F.Cu") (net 47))
 (segment (start 36.449 131.445) (end 41.91 131.445) (width 0.25) (layer "F.Cu") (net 48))
 (segment (start 36.449 128.905) (end 41.91 128.905) (width 0.25) (layer "F.Cu") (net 49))
 (segment (start 36.449 126.365) (end 41.91 126.365) (width 0.25) (layer "F.Cu") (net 50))
 (segment (start 36.449 187.325) (end 41.91 187.325) (width 0.25) (layer "F.Cu") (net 26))
 (segment (start 36.449 184.785) (end 41.91 184.785) (width 0.25) (layer "F.Cu") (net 27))
 (segment (start 36.449 182.245) (end 41.91 182.245) (width 0.25) (layer "F.Cu") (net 28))
 (segment (start 36.449 179.705) (end 41.91 179.705) (width 0.25) (layer "F.Cu") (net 29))
 (segment (start 36.449 177.165) (end 41.91 177.165) (width 0.25) (layer "F.Cu") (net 30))
 (segment (start 36.449 174.625) (end 41.91 174.625) (width 0.25) (layer "F.Cu") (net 31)))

